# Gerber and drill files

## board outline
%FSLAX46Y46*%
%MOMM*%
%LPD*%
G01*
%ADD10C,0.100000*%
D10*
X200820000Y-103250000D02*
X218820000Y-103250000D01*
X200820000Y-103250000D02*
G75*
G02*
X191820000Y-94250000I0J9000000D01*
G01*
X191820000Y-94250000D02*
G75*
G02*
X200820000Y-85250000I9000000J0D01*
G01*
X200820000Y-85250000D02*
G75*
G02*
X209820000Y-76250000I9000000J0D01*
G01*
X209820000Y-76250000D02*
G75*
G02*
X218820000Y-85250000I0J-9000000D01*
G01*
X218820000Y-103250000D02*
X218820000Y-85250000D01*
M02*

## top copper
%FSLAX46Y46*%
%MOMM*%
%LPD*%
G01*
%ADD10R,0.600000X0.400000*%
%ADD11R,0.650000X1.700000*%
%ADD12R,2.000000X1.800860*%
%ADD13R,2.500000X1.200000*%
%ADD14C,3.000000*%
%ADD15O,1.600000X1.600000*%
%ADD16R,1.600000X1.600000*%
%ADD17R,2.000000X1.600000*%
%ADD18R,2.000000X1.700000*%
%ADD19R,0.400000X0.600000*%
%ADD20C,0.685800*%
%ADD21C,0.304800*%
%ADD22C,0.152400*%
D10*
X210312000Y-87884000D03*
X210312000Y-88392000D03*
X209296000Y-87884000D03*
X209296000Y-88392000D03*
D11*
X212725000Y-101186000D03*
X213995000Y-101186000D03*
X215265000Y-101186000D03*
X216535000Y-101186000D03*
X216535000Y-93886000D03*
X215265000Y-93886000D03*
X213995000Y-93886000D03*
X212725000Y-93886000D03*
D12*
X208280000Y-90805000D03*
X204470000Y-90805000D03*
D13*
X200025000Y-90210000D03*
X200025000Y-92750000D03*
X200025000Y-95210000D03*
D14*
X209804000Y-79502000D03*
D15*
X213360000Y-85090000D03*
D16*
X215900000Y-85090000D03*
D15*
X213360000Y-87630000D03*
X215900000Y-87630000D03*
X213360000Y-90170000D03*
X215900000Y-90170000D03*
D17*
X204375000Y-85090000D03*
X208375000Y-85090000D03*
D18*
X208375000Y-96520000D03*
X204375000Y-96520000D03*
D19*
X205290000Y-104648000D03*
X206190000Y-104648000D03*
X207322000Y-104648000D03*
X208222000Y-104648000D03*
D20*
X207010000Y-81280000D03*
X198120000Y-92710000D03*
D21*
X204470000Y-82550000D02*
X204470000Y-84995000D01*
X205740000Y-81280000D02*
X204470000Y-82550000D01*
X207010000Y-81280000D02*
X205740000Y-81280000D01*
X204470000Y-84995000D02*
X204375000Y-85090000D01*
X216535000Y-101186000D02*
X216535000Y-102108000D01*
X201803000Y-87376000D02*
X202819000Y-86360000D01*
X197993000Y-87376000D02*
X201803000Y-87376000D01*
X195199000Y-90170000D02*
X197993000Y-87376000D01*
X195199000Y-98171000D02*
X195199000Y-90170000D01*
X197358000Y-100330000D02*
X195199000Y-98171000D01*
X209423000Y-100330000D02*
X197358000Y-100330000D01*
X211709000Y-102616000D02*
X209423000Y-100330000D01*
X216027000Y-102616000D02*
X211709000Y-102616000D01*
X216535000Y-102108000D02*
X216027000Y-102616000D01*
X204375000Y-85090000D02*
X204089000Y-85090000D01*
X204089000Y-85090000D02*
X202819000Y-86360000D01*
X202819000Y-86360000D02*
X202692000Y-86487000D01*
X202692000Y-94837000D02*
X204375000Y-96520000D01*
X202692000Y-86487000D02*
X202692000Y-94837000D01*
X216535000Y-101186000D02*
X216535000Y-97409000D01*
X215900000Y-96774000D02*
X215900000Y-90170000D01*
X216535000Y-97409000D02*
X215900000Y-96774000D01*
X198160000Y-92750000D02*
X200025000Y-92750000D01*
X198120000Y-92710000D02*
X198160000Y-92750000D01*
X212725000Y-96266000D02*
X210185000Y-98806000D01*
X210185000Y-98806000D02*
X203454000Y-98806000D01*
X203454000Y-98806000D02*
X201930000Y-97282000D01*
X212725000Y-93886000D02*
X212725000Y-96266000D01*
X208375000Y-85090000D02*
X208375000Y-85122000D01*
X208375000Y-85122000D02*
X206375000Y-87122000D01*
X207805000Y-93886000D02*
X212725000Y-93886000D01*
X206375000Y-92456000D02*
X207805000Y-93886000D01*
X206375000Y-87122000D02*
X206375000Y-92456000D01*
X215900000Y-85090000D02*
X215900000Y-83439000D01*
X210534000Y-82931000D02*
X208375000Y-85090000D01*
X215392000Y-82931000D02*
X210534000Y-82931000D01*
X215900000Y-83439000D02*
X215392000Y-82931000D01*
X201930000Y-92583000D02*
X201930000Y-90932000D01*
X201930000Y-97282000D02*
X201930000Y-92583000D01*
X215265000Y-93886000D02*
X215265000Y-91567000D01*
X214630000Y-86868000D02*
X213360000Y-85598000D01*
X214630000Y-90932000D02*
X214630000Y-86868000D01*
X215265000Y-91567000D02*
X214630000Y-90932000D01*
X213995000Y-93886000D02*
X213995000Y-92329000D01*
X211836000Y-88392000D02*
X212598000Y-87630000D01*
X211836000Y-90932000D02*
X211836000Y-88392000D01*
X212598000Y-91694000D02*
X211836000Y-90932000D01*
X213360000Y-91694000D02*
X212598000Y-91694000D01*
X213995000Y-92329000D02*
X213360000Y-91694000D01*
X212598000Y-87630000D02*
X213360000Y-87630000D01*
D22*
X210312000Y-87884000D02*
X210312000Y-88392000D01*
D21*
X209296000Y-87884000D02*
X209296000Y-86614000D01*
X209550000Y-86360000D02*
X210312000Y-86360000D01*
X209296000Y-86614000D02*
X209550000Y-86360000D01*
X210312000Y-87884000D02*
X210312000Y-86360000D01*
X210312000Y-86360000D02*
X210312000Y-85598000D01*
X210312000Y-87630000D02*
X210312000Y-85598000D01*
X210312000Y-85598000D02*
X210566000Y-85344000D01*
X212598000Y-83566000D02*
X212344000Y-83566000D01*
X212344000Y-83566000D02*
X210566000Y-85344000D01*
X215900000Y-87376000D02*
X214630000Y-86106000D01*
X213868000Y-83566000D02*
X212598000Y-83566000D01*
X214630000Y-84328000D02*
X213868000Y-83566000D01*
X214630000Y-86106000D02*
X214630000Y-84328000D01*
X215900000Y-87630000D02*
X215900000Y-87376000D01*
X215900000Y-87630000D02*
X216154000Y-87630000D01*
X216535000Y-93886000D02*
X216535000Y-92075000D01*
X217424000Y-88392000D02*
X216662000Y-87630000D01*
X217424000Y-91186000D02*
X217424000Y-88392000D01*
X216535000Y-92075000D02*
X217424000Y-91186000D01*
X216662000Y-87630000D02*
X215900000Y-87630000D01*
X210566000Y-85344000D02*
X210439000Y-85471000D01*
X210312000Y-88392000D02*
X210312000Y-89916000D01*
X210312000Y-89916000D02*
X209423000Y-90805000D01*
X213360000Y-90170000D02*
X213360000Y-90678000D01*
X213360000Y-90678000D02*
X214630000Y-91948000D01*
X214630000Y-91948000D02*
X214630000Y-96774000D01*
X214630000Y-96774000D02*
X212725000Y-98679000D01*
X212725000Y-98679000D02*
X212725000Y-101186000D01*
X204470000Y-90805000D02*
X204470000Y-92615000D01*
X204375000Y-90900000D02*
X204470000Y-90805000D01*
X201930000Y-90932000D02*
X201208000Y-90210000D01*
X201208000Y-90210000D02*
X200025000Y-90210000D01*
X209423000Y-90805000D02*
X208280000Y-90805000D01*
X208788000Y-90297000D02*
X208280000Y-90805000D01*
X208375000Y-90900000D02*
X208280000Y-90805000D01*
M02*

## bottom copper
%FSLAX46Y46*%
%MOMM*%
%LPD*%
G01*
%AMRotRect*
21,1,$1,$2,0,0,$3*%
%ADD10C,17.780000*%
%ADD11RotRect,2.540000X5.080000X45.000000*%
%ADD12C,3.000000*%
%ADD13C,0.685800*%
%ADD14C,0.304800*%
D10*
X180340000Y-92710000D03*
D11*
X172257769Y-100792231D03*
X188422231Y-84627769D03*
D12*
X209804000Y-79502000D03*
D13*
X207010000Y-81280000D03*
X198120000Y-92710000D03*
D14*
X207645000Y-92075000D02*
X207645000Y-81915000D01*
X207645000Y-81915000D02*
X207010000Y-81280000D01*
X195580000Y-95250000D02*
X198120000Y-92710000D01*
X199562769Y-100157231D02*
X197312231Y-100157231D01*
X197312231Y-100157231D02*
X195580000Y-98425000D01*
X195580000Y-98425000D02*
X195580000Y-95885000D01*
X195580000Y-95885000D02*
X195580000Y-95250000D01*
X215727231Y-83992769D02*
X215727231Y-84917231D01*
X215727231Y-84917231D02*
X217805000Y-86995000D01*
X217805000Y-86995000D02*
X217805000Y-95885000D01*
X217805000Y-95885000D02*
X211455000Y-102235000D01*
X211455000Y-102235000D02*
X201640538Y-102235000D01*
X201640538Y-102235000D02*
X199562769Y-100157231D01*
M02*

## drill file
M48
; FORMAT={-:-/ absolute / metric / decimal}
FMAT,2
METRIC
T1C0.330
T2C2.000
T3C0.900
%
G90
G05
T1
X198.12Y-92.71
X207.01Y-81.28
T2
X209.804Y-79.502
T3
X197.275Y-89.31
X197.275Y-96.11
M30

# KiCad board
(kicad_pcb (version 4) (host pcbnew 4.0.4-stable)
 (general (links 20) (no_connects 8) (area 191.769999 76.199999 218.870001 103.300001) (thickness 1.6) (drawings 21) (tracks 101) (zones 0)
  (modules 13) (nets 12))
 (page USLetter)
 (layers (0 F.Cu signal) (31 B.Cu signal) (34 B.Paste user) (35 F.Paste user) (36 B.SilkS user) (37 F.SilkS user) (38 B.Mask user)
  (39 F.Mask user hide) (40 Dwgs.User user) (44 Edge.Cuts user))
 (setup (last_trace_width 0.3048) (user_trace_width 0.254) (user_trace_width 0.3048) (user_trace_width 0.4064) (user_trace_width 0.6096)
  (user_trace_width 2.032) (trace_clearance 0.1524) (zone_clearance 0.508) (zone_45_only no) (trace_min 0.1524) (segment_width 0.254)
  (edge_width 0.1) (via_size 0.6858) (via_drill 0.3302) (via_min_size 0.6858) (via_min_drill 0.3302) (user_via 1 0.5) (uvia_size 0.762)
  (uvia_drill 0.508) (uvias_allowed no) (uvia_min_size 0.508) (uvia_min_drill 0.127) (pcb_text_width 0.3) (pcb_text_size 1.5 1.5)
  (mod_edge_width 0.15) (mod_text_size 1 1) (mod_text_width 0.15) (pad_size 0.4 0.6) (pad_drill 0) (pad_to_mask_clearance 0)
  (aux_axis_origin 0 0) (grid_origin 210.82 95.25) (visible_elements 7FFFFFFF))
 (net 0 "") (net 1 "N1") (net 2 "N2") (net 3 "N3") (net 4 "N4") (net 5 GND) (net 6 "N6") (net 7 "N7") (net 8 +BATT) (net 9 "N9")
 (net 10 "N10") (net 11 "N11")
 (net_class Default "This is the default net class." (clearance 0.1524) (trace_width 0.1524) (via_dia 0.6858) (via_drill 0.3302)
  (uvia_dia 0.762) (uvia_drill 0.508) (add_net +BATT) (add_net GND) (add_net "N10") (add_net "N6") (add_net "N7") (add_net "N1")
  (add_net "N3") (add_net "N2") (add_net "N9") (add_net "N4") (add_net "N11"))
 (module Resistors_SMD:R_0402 (layer F.Cu) (at 210.312 88.138 270)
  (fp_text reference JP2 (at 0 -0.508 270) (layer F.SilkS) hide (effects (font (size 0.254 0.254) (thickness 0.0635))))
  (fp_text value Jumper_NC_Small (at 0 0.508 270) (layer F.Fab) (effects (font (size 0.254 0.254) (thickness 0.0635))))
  (pad 1 smd rect (at -0.254 0 270) (size 0.4 0.6) (layers F.Cu F.Paste F.Mask) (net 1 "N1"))
  (pad 1 smd rect (at 0.254 0 270) (size 0.4 0.6) (layers F.Cu F.Paste F.Mask) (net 1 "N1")))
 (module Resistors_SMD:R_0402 (layer F.Cu) (at 209.296 88.138 270)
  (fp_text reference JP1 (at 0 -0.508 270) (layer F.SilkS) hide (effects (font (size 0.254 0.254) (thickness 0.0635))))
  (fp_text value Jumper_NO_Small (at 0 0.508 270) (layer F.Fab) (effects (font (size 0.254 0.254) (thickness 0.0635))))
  (pad 1 smd rect (at -0.254 0 270) (size 0.4 0.6) (layers F.Cu F.Paste F.Mask) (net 1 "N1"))
  (pad 2 smd rect (at 0.254 0 270) (size 0.4 0.6) (layers F.Cu F.Paste F.Mask) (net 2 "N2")))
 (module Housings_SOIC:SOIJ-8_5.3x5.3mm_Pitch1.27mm (layer F.Cu) (at 214.63 97.536 90)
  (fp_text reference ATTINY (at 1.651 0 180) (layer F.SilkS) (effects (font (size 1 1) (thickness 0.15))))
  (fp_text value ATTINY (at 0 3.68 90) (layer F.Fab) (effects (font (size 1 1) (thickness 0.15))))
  (pad 1 smd rect (at -3.65 -1.905 90) (size 1.7 0.65) (layers F.Cu F.Paste F.Mask) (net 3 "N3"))
  (pad 2 smd rect (at -3.65 -0.635 90) (size 1.7 0.65) (layers F.Cu F.Paste F.Mask) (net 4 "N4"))
  (pad 3 smd rect (at -3.65 0.635 90) (size 1.7 0.65) (layers F.Cu F.Paste F.Mask))
  (pad 4 smd rect (at -3.65 1.905 90) (size 1.7 0.65) (layers F.Cu F.Paste F.Mask) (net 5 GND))
  (pad 5 smd rect (at 3.65 1.905 90) (size 1.7 0.65) (layers F.Cu F.Paste F.Mask) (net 1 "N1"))
  (pad 6 smd rect (at 3.65 0.635 90) (size 1.7 0.65) (layers F.Cu F.Paste F.Mask) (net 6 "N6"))
  (pad 7 smd rect (at 3.65 -0.635 90) (size 1.7 0.65) (layers F.Cu F.Paste F.Mask) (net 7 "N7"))
  (pad 8 smd rect (at 3.65 -1.905 90) (size 1.7 0.65) (layers F.Cu F.Paste F.Mask) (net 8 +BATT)))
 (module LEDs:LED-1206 (layer F.Cu) (at 206.375 90.805)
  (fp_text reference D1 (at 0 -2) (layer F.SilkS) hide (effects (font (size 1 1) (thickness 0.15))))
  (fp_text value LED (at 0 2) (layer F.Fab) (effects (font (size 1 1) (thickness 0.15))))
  (pad 2 smd rect (at 1.905 0 180) (size 2 1.80086) (layers F.Cu F.Paste F.Mask) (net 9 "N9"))
  (pad 1 smd rect (at -1.905 0 180) (size 2 1.80086) (layers F.Cu F.Paste F.Mask) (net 2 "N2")))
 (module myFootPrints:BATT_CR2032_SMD (layer B.Cu) (at 180.34 92.71 45)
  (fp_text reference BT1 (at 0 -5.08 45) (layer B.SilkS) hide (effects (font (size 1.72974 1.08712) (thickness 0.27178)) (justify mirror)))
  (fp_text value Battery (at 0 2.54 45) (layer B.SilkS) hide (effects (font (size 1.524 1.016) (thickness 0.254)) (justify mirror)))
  (pad 2 smd circle (at 0 0 45) (size 17.78 17.78) (layers B.Cu B.Paste B.Mask) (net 5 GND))
  (pad 1 smd rect (at -11.43 0 45) (size 2.54 5.08) (layers B.Cu B.Paste B.Mask) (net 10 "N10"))
  (pad 1 smd rect (at 11.43 0 45) (size 2.54 5.08) (layers B.Cu B.Paste B.Mask) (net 10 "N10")))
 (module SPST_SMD (layer F.Cu) (at 200.025 92.71 270)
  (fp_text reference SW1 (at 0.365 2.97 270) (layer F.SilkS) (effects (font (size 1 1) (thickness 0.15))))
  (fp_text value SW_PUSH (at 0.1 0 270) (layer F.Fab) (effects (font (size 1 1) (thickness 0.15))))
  (pad "" np_thru_hole circle (at 3.4 2.75 270) (size 0.9 0.9) (drill 0.9) (layers *.Cu *.Mask))
  (pad 1 smd rect (at -2.5 0 270) (size 1.2 2.5) (layers F.Cu F.Paste F.Mask) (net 4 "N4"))
  (pad 2 smd rect (at 0.04 0 270) (size 1.2 2.5) (layers F.Cu F.Paste F.Mask) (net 5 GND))
  (pad 3 smd rect (at 2.5 0 270) (size 1.2 2.5) (layers F.Cu F.Paste F.Mask))
  (pad "" np_thru_hole circle (at -3.4 2.75 270) (size 0.9 0.9) (drill 0.9) (layers *.Cu *.Mask)))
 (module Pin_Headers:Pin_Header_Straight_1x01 (layer F.Cu) (at 209.804 79.502)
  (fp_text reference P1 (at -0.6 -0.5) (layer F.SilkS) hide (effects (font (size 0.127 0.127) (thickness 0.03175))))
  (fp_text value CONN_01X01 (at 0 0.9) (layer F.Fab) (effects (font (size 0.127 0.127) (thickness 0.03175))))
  (pad "" thru_hole circle (at 0 0) (size 3 3) (drill 2) (layers *.Cu *.Mask)))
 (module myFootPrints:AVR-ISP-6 (layer F.Cu) (at 213.36 85.09)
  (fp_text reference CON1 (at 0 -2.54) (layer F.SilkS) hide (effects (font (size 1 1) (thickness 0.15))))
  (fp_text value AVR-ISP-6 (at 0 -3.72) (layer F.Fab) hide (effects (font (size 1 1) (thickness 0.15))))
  (pad 1 smd oval (at 0 0) (size 1.6 1.6) (layers F.Cu F.Paste F.Mask) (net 6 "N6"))
  (pad 2 smd rect (at 2.54 0) (size 1.6 1.6) (layers F.Cu F.Paste F.Mask) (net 8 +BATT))
  (pad 3 smd oval (at 0 2.54) (size 1.6 1.6) (layers F.Cu F.Paste F.Mask) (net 7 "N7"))
  (pad 4 smd oval (at 2.54 2.54) (size 1.6 1.6) (layers F.Cu F.Paste F.Mask) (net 1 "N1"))
  (pad 5 smd oval (at 0 5.08) (size 1.6 1.6) (layers F.Cu F.Paste F.Mask) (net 3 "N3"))
  (pad 6 smd oval (at 2.54 5.08) (size 1.6 1.6) (layers F.Cu F.Paste F.Mask) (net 5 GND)))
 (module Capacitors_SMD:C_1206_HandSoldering (layer F.Cu) (at 206.375 85.09)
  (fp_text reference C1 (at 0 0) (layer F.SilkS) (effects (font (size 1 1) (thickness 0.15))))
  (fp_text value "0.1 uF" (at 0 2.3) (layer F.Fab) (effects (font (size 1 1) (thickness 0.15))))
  (pad 1 smd rect (at -2 0) (size 2 1.6) (layers F.Cu F.Paste F.Mask) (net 5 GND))
  (pad 2 smd rect (at 2 0) (size 2 1.6) (layers F.Cu F.Paste F.Mask) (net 8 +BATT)))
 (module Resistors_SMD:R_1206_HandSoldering (layer F.Cu) (at 206.375 96.52 180)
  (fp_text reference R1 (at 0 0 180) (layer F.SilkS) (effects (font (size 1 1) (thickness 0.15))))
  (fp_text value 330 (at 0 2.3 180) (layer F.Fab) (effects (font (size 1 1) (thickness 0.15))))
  (pad 1 smd rect (at -2 0 180) (size 2 1.7) (layers F.Cu F.Paste F.Mask) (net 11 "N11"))
  (pad 2 smd rect (at 2 0 180) (size 2 1.7) (layers F.Cu F.Paste F.Mask) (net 5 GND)))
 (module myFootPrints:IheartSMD (layer F.Cu) (at 203.835 100.33)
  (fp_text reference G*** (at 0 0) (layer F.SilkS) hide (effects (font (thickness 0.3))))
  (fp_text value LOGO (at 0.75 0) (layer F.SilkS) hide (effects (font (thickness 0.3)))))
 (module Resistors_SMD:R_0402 (layer F.Cu) (at 205.74 104.648)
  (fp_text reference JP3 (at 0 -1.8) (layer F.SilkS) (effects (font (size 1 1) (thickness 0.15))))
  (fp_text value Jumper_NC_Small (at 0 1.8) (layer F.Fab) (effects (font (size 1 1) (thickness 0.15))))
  (pad 1 smd rect (at -0.45 0) (size 0.4 0.6) (layers F.Cu F.Paste F.Mask) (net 2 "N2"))
  (pad 2 smd rect (at 0.45 0) (size 0.4 0.6) (layers F.Cu F.Paste F.Mask)))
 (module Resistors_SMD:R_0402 (layer F.Cu) (at 207.772 104.648)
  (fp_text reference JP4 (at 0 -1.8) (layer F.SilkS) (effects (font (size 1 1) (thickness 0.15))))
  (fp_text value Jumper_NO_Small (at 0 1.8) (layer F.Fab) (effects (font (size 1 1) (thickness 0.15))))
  (pad 1 smd rect (at -0.45 0) (size 0.4 0.6) (layers F.Cu F.Paste F.Mask) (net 9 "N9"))
  (pad 2 smd rect (at 0.45 0) (size 0.4 0.6) (layers F.Cu F.Paste F.Mask) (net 11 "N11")))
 (gr_line (start 200.82 103.25) (end 218.82 103.25) (angle 90) (layer Edge.Cuts) (width 0.1))
 (gr_arc (start 200.82 94.25) (end 200.82 103.25) (angle 90) (layer Edge.Cuts) (width 0.1))
 (gr_arc (start 200.82 94.25) (end 191.82 94.25) (angle 90) (layer Edge.Cuts) (width 0.1))
 (gr_arc (start 209.82 85.25) (end 200.82 85.25) (angle 90) (layer Edge.Cuts) (width 0.1))
 (gr_arc (start 209.82 85.25) (end 209.82 76.25) (angle 90) (layer Edge.Cuts) (width 0.1))
 (gr_line (start 218.82 103.25) (end 218.82 85.25) (angle 90) (layer Edge.Cuts) (width 0.1))
 (segment (start 207.645 92.075) (end 207.645 81.915) (width 0.3048) (layer B.Cu) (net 5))
 (segment (start 204.47 82.55) (end 204.47 84.995) (width 0.3048) (layer F.Cu) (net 5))
 (segment (start 205.74 81.28) (end 204.47 82.55) (width 0.3048) (layer F.Cu) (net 5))
 (segment (start 207.01 81.28) (end 205.74 81.28) (width 0.3048) (layer F.Cu) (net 5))
 (via (at 207.01 81.28) (size 0.6858) (drill 0.3302) (layers F.Cu B.Cu) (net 5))
 (segment (start 207.645 81.915) (end 207.01 81.28) (width 0.3048) (layer B.Cu) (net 5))
 (segment (start 204.47 84.995) (end 204.375 85.09) (width 0.3048) (layer F.Cu) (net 5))
 (segment (start 216.535 101.186) (end 216.535 102.108) (width 0.3048) (layer F.Cu) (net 5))
 (segment (start 201.803 87.376) (end 202.819 86.36) (width 0.3048) (layer F.Cu) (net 5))
 (segment (start 197.993 87.376) (end 201.803 87.376) (width 0.3048) (layer F.Cu) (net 5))
 (segment (start 195.199 90.17) (end 197.993 87.376) (width 0.3048) (layer F.Cu) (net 5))
 (segment (start 195.199 98.171) (end 195.199 90.17) (width 0.3048) (layer F.Cu) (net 5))
 (segment (start 197.358 100.33) (end 195.199 98.171) (width 0.3048) (layer F.Cu) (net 5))
 (segment (start 209.423 100.33) (end 197.358 100.33) (width 0.3048) (layer F.Cu) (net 5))
 (segment (start 211.709 102.616) (end 209.423 100.33) (width 0.3048) (layer F.Cu) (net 5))
 (segment (start 216.027 102.616) (end 211.709 102.616) (width 0.3048) (layer F.Cu) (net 5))
 (segment (start 216.535 102.108) (end 216.027 102.616) (width 0.3048) (layer F.Cu) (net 5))
 (segment (start 204.375 85.09) (end 204.089 85.09) (width 0.3048) (layer F.Cu) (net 5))
 (segment (start 204.089 85.09) (end 202.819 86.36) (width 0.3048) (layer F.Cu) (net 5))
 (segment (start 202.819 86.36) (end 202.692 86.487) (width 0.3048) (layer F.Cu) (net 5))
 (segment (start 202.692 94.837) (end 204.375 96.52) (width 0.3048) (layer F.Cu) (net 5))
 (segment (start 202.692 86.487) (end 202.692 94.837) (width 0.3048) (layer F.Cu) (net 5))
 (segment (start 216.535 101.186) (end 216.535 97.409) (width 0.3048) (layer F.Cu) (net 5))
 (segment (start 215.9 96.774) (end 215.9 90.17) (width 0.3048) (layer F.Cu) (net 5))
 (segment (start 216.535 97.409) (end 215.9 96.774) (width 0.3048) (layer F.Cu) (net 5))
 (segment (start 195.58 95.25) (end 198.12 92.71) (width 0.3048) (layer B.Cu) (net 5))
 (segment (start 198.16 92.75) (end 200.025 92.75) (width 0.3048) (layer F.Cu) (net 5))
 (via (at 198.12 92.71) (size 0.6858) (drill 0.3302) (layers F.Cu B.Cu) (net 5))
 (segment (start 198.12 92.71) (end 198.16 92.75) (width 0.3048) (layer F.Cu) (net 5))
 (segment (start 199.562769 100.157231) (end 197.312231 100.157231) (width 0.3048) (layer B.Cu) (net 5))
 (segment (start 197.312231 100.157231) (end 195.58 98.425) (width 0.3048) (layer B.Cu) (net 5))
 (segment (start 195.58 98.425) (end 195.58 95.885) (width 0.3048) (layer B.Cu) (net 5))
 (segment (start 195.58 95.885) (end 195.58 95.25) (width 0.3048) (layer B.Cu) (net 5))
 (segment (start 215.727231 83.992769) (end 215.727231 84.917231) (width 0.3048) (layer B.Cu) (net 5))
 (segment (start 215.727231 84.917231) (end 217.805 86.995) (width 0.3048) (layer B.Cu) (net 5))
 (segment (start 217.805 86.995) (end 217.805 95.885) (width 0.3048) (layer B.Cu) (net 5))
 (segment (start 217.805 95.885) (end 211.455 102.235) (width 0.3048) (layer B.Cu) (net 5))
 (segment (start 211.455 102.235) (end 201.640538 102.235) (width 0.3048) (layer B.Cu) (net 5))
 (segment (start 201.640538 102.235) (end 199.562769 100.157231) (width 0.3048) (layer B.Cu) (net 5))
 (segment (start 212.725 96.266) (end 210.185 98.806) (width 0.3048) (layer F.Cu) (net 8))
 (segment (start 210.185 98.806) (end 203.454 98.806) (width 0.3048) (layer F.Cu) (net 8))
 (segment (start 203.454 98.806) (end 201.93 97.282) (width 0.3048) (layer F.Cu) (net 8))
 (segment (start 212.725 93.886) (end 212.725 96.266) (width 0.3048) (layer F.Cu) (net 8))
 (segment (start 208.375 85.09) (end 208.375 85.122) (width 0.3048) (layer F.Cu) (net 8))
 (segment (start 208.375 85.122) (end 206.375 87.122) (width 0.3048) (layer F.Cu) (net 8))
 (segment (start 207.805 93.886) (end 212.725 93.886) (width 0.3048) (layer F.Cu) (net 8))
 (segment (start 206.375 92.456) (end 207.805 93.886) (width 0.3048) (layer F.Cu) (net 8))
 (segment (start 206.375 87.122) (end 206.375 92.456) (width 0.3048) (layer F.Cu) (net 8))
 (segment (start 215.9 85.09) (end 215.9 83.439) (width 0.3048) (layer F.Cu) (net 8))
 (segment (start 210.534 82.931) (end 208.375 85.09) (width 0.3048) (layer F.Cu) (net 8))
 (segment (start 215.392 82.931) (end 210.534 82.931) (width 0.3048) (layer F.Cu) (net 8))
 (segment (start 215.9 83.439) (end 215.392 82.931) (width 0.3048) (layer F.Cu) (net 8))
 (segment (start 201.93 92.583) (end 201.93 90.932) (width 0.3048) (layer F.Cu) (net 8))
 (segment (start 201.93 97.282) (end 201.93 92.583) (width 0.3048) (layer F.Cu) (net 8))
 (segment (start 215.265 93.886) (end 215.265 91.567) (width 0.3048) (layer F.Cu) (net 6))
 (segment (start 214.63 86.868) (end 213.36 85.598) (width 0.3048) (layer F.Cu) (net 6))
 (segment (start 214.63 90.932) (end 214.63 86.868) (width 0.3048) (layer F.Cu) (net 6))
 (segment (start 215.265 91.567) (end 214.63 90.932) (width 0.3048) (layer F.Cu) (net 6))
 (segment (start 213.995 93.886) (end 213.995 92.329) (width 0.3048) (layer F.Cu) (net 7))
 (segment (start 211.836 88.392) (end 212.598 87.63) (width 0.3048) (layer F.Cu) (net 7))
 (segment (start 211.836 90.932) (end 211.836 88.392) (width 0.3048) (layer F.Cu) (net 7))
 (segment (start 212.598 91.694) (end 211.836 90.932) (width 0.3048) (layer F.Cu) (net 7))
 (segment (start 213.36 91.694) (end 212.598 91.694) (width 0.3048) (layer F.Cu) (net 7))
 (segment (start 213.995 92.329) (end 213.36 91.694) (width 0.3048) (layer F.Cu) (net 7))
 (segment (start 212.598 87.63) (end 213.36 87.63) (width 0.3048) (layer F.Cu) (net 7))
 (segment (start 210.312 87.884) (end 210.312 88.392) (width 0.1524) (layer F.Cu) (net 1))
 (segment (start 209.296 87.884) (end 209.296 86.614) (width 0.3048) (layer F.Cu) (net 1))
 (segment (start 209.55 86.36) (end 210.312 86.36) (width 0.3048) (layer F.Cu) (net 1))
 (segment (start 209.296 86.614) (end 209.55 86.36) (width 0.3048) (layer F.Cu) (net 1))
 (segment (start 210.312 87.884) (end 210.312 86.36) (width 0.3048) (layer F.Cu) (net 1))
 (segment (start 210.312 86.36) (end 210.312 85.598) (width 0.3048) (layer F.Cu) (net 1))
 (segment (start 210.312 87.63) (end 210.312 85.598) (width 0.3048) (layer F.Cu) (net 1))
 (segment (start 210.312 85.598) (end 210.566 85.344) (width 0.3048) (layer F.Cu) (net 1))
 (segment (start 212.598 83.566) (end 212.344 83.566) (width 0.3048) (layer F.Cu) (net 1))
 (segment (start 212.344 83.566) (end 210.566 85.344) (width 0.3048) (layer F.Cu) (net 1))
 (segment (start 215.9 87.376) (end 214.63 86.106) (width 0.3048) (layer F.Cu) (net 1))
 (segment (start 213.868 83.566) (end 212.598 83.566) (width 0.3048) (layer F.Cu) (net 1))
 (segment (start 214.63 84.328) (end 213.868 83.566) (width 0.3048) (layer F.Cu) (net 1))
 (segment (start 214.63 86.106) (end 214.63 84.328) (width 0.3048) (layer F.Cu) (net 1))
 (segment (start 215.9 87.63) (end 215.9 87.376) (width 0.3048) (layer F.Cu) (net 1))
 (segment (start 215.9 87.63) (end 216.154 87.63) (width 0.3048) (layer F.Cu) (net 1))
 (segment (start 216.535 93.886) (end 216.535 92.075) (width 0.3048) (layer F.Cu) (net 1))
 (segment (start 217.424 88.392) (end 216.662 87.63) (width 0.3048) (layer F.Cu) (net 1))
 (segment (start 217.424 91.186) (end 217.424 88.392) (width 0.3048) (layer F.Cu) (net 1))
 (segment (start 216.535 92.075) (end 217.424 91.186) (width 0.3048) (layer F.Cu) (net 1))
 (segment (start 216.662 87.63) (end 215.9 87.63) (width 0.3048) (layer F.Cu) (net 1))
 (segment (start 210.566 85.344) (end 210.439 85.471) (width 0.3048) (layer F.Cu) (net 1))
 (segment (start 210.312 88.392) (end 210.312 89.916) (width 0.3048) (layer F.Cu) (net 1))
 (segment (start 210.312 89.916) (end 209.423 90.805) (width 0.3048) (layer F.Cu) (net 1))
 (segment (start 213.36 90.17) (end 213.36 90.678) (width 0.3048) (layer F.Cu) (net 3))
 (segment (start 213.36 90.678) (end 214.63 91.948) (width 0.3048) (layer F.Cu) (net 3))
 (segment (start 214.63 91.948) (end 214.63 96.774) (width 0.3048) (layer F.Cu) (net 3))
 (segment (start 214.63 96.774) (end 212.725 98.679) (width 0.3048) (layer F.Cu) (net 3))
 (segment (start 212.725 98.679) (end 212.725 101.186) (width 0.3048) (layer F.Cu) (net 3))
 (segment (start 204.47 90.805) (end 204.47 92.615) (width 0.3048) (layer F.Cu) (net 2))
 (segment (start 204.375 90.9) (end 204.47 90.805) (width 0.3048) (layer F.Cu) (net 2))
 (segment (start 201.93 90.932) (end 201.208 90.21) (width 0.3048) (layer F.Cu) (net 4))
 (segment (start 201.208 90.21) (end 200.025 90.21) (width 0.3048) (layer F.Cu) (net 4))
 (segment (start 209.423 90.805) (end 208.28 90.805) (width 0.3048) (layer F.Cu) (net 9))
 (segment (start 208.788 90.297) (end 208.28 90.805) (width 0.3048) (layer F.Cu) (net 9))
 (segment (start 208.375 90.9) (end 208.28 90.805) (width 0.3048) (layer F.Cu) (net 9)))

